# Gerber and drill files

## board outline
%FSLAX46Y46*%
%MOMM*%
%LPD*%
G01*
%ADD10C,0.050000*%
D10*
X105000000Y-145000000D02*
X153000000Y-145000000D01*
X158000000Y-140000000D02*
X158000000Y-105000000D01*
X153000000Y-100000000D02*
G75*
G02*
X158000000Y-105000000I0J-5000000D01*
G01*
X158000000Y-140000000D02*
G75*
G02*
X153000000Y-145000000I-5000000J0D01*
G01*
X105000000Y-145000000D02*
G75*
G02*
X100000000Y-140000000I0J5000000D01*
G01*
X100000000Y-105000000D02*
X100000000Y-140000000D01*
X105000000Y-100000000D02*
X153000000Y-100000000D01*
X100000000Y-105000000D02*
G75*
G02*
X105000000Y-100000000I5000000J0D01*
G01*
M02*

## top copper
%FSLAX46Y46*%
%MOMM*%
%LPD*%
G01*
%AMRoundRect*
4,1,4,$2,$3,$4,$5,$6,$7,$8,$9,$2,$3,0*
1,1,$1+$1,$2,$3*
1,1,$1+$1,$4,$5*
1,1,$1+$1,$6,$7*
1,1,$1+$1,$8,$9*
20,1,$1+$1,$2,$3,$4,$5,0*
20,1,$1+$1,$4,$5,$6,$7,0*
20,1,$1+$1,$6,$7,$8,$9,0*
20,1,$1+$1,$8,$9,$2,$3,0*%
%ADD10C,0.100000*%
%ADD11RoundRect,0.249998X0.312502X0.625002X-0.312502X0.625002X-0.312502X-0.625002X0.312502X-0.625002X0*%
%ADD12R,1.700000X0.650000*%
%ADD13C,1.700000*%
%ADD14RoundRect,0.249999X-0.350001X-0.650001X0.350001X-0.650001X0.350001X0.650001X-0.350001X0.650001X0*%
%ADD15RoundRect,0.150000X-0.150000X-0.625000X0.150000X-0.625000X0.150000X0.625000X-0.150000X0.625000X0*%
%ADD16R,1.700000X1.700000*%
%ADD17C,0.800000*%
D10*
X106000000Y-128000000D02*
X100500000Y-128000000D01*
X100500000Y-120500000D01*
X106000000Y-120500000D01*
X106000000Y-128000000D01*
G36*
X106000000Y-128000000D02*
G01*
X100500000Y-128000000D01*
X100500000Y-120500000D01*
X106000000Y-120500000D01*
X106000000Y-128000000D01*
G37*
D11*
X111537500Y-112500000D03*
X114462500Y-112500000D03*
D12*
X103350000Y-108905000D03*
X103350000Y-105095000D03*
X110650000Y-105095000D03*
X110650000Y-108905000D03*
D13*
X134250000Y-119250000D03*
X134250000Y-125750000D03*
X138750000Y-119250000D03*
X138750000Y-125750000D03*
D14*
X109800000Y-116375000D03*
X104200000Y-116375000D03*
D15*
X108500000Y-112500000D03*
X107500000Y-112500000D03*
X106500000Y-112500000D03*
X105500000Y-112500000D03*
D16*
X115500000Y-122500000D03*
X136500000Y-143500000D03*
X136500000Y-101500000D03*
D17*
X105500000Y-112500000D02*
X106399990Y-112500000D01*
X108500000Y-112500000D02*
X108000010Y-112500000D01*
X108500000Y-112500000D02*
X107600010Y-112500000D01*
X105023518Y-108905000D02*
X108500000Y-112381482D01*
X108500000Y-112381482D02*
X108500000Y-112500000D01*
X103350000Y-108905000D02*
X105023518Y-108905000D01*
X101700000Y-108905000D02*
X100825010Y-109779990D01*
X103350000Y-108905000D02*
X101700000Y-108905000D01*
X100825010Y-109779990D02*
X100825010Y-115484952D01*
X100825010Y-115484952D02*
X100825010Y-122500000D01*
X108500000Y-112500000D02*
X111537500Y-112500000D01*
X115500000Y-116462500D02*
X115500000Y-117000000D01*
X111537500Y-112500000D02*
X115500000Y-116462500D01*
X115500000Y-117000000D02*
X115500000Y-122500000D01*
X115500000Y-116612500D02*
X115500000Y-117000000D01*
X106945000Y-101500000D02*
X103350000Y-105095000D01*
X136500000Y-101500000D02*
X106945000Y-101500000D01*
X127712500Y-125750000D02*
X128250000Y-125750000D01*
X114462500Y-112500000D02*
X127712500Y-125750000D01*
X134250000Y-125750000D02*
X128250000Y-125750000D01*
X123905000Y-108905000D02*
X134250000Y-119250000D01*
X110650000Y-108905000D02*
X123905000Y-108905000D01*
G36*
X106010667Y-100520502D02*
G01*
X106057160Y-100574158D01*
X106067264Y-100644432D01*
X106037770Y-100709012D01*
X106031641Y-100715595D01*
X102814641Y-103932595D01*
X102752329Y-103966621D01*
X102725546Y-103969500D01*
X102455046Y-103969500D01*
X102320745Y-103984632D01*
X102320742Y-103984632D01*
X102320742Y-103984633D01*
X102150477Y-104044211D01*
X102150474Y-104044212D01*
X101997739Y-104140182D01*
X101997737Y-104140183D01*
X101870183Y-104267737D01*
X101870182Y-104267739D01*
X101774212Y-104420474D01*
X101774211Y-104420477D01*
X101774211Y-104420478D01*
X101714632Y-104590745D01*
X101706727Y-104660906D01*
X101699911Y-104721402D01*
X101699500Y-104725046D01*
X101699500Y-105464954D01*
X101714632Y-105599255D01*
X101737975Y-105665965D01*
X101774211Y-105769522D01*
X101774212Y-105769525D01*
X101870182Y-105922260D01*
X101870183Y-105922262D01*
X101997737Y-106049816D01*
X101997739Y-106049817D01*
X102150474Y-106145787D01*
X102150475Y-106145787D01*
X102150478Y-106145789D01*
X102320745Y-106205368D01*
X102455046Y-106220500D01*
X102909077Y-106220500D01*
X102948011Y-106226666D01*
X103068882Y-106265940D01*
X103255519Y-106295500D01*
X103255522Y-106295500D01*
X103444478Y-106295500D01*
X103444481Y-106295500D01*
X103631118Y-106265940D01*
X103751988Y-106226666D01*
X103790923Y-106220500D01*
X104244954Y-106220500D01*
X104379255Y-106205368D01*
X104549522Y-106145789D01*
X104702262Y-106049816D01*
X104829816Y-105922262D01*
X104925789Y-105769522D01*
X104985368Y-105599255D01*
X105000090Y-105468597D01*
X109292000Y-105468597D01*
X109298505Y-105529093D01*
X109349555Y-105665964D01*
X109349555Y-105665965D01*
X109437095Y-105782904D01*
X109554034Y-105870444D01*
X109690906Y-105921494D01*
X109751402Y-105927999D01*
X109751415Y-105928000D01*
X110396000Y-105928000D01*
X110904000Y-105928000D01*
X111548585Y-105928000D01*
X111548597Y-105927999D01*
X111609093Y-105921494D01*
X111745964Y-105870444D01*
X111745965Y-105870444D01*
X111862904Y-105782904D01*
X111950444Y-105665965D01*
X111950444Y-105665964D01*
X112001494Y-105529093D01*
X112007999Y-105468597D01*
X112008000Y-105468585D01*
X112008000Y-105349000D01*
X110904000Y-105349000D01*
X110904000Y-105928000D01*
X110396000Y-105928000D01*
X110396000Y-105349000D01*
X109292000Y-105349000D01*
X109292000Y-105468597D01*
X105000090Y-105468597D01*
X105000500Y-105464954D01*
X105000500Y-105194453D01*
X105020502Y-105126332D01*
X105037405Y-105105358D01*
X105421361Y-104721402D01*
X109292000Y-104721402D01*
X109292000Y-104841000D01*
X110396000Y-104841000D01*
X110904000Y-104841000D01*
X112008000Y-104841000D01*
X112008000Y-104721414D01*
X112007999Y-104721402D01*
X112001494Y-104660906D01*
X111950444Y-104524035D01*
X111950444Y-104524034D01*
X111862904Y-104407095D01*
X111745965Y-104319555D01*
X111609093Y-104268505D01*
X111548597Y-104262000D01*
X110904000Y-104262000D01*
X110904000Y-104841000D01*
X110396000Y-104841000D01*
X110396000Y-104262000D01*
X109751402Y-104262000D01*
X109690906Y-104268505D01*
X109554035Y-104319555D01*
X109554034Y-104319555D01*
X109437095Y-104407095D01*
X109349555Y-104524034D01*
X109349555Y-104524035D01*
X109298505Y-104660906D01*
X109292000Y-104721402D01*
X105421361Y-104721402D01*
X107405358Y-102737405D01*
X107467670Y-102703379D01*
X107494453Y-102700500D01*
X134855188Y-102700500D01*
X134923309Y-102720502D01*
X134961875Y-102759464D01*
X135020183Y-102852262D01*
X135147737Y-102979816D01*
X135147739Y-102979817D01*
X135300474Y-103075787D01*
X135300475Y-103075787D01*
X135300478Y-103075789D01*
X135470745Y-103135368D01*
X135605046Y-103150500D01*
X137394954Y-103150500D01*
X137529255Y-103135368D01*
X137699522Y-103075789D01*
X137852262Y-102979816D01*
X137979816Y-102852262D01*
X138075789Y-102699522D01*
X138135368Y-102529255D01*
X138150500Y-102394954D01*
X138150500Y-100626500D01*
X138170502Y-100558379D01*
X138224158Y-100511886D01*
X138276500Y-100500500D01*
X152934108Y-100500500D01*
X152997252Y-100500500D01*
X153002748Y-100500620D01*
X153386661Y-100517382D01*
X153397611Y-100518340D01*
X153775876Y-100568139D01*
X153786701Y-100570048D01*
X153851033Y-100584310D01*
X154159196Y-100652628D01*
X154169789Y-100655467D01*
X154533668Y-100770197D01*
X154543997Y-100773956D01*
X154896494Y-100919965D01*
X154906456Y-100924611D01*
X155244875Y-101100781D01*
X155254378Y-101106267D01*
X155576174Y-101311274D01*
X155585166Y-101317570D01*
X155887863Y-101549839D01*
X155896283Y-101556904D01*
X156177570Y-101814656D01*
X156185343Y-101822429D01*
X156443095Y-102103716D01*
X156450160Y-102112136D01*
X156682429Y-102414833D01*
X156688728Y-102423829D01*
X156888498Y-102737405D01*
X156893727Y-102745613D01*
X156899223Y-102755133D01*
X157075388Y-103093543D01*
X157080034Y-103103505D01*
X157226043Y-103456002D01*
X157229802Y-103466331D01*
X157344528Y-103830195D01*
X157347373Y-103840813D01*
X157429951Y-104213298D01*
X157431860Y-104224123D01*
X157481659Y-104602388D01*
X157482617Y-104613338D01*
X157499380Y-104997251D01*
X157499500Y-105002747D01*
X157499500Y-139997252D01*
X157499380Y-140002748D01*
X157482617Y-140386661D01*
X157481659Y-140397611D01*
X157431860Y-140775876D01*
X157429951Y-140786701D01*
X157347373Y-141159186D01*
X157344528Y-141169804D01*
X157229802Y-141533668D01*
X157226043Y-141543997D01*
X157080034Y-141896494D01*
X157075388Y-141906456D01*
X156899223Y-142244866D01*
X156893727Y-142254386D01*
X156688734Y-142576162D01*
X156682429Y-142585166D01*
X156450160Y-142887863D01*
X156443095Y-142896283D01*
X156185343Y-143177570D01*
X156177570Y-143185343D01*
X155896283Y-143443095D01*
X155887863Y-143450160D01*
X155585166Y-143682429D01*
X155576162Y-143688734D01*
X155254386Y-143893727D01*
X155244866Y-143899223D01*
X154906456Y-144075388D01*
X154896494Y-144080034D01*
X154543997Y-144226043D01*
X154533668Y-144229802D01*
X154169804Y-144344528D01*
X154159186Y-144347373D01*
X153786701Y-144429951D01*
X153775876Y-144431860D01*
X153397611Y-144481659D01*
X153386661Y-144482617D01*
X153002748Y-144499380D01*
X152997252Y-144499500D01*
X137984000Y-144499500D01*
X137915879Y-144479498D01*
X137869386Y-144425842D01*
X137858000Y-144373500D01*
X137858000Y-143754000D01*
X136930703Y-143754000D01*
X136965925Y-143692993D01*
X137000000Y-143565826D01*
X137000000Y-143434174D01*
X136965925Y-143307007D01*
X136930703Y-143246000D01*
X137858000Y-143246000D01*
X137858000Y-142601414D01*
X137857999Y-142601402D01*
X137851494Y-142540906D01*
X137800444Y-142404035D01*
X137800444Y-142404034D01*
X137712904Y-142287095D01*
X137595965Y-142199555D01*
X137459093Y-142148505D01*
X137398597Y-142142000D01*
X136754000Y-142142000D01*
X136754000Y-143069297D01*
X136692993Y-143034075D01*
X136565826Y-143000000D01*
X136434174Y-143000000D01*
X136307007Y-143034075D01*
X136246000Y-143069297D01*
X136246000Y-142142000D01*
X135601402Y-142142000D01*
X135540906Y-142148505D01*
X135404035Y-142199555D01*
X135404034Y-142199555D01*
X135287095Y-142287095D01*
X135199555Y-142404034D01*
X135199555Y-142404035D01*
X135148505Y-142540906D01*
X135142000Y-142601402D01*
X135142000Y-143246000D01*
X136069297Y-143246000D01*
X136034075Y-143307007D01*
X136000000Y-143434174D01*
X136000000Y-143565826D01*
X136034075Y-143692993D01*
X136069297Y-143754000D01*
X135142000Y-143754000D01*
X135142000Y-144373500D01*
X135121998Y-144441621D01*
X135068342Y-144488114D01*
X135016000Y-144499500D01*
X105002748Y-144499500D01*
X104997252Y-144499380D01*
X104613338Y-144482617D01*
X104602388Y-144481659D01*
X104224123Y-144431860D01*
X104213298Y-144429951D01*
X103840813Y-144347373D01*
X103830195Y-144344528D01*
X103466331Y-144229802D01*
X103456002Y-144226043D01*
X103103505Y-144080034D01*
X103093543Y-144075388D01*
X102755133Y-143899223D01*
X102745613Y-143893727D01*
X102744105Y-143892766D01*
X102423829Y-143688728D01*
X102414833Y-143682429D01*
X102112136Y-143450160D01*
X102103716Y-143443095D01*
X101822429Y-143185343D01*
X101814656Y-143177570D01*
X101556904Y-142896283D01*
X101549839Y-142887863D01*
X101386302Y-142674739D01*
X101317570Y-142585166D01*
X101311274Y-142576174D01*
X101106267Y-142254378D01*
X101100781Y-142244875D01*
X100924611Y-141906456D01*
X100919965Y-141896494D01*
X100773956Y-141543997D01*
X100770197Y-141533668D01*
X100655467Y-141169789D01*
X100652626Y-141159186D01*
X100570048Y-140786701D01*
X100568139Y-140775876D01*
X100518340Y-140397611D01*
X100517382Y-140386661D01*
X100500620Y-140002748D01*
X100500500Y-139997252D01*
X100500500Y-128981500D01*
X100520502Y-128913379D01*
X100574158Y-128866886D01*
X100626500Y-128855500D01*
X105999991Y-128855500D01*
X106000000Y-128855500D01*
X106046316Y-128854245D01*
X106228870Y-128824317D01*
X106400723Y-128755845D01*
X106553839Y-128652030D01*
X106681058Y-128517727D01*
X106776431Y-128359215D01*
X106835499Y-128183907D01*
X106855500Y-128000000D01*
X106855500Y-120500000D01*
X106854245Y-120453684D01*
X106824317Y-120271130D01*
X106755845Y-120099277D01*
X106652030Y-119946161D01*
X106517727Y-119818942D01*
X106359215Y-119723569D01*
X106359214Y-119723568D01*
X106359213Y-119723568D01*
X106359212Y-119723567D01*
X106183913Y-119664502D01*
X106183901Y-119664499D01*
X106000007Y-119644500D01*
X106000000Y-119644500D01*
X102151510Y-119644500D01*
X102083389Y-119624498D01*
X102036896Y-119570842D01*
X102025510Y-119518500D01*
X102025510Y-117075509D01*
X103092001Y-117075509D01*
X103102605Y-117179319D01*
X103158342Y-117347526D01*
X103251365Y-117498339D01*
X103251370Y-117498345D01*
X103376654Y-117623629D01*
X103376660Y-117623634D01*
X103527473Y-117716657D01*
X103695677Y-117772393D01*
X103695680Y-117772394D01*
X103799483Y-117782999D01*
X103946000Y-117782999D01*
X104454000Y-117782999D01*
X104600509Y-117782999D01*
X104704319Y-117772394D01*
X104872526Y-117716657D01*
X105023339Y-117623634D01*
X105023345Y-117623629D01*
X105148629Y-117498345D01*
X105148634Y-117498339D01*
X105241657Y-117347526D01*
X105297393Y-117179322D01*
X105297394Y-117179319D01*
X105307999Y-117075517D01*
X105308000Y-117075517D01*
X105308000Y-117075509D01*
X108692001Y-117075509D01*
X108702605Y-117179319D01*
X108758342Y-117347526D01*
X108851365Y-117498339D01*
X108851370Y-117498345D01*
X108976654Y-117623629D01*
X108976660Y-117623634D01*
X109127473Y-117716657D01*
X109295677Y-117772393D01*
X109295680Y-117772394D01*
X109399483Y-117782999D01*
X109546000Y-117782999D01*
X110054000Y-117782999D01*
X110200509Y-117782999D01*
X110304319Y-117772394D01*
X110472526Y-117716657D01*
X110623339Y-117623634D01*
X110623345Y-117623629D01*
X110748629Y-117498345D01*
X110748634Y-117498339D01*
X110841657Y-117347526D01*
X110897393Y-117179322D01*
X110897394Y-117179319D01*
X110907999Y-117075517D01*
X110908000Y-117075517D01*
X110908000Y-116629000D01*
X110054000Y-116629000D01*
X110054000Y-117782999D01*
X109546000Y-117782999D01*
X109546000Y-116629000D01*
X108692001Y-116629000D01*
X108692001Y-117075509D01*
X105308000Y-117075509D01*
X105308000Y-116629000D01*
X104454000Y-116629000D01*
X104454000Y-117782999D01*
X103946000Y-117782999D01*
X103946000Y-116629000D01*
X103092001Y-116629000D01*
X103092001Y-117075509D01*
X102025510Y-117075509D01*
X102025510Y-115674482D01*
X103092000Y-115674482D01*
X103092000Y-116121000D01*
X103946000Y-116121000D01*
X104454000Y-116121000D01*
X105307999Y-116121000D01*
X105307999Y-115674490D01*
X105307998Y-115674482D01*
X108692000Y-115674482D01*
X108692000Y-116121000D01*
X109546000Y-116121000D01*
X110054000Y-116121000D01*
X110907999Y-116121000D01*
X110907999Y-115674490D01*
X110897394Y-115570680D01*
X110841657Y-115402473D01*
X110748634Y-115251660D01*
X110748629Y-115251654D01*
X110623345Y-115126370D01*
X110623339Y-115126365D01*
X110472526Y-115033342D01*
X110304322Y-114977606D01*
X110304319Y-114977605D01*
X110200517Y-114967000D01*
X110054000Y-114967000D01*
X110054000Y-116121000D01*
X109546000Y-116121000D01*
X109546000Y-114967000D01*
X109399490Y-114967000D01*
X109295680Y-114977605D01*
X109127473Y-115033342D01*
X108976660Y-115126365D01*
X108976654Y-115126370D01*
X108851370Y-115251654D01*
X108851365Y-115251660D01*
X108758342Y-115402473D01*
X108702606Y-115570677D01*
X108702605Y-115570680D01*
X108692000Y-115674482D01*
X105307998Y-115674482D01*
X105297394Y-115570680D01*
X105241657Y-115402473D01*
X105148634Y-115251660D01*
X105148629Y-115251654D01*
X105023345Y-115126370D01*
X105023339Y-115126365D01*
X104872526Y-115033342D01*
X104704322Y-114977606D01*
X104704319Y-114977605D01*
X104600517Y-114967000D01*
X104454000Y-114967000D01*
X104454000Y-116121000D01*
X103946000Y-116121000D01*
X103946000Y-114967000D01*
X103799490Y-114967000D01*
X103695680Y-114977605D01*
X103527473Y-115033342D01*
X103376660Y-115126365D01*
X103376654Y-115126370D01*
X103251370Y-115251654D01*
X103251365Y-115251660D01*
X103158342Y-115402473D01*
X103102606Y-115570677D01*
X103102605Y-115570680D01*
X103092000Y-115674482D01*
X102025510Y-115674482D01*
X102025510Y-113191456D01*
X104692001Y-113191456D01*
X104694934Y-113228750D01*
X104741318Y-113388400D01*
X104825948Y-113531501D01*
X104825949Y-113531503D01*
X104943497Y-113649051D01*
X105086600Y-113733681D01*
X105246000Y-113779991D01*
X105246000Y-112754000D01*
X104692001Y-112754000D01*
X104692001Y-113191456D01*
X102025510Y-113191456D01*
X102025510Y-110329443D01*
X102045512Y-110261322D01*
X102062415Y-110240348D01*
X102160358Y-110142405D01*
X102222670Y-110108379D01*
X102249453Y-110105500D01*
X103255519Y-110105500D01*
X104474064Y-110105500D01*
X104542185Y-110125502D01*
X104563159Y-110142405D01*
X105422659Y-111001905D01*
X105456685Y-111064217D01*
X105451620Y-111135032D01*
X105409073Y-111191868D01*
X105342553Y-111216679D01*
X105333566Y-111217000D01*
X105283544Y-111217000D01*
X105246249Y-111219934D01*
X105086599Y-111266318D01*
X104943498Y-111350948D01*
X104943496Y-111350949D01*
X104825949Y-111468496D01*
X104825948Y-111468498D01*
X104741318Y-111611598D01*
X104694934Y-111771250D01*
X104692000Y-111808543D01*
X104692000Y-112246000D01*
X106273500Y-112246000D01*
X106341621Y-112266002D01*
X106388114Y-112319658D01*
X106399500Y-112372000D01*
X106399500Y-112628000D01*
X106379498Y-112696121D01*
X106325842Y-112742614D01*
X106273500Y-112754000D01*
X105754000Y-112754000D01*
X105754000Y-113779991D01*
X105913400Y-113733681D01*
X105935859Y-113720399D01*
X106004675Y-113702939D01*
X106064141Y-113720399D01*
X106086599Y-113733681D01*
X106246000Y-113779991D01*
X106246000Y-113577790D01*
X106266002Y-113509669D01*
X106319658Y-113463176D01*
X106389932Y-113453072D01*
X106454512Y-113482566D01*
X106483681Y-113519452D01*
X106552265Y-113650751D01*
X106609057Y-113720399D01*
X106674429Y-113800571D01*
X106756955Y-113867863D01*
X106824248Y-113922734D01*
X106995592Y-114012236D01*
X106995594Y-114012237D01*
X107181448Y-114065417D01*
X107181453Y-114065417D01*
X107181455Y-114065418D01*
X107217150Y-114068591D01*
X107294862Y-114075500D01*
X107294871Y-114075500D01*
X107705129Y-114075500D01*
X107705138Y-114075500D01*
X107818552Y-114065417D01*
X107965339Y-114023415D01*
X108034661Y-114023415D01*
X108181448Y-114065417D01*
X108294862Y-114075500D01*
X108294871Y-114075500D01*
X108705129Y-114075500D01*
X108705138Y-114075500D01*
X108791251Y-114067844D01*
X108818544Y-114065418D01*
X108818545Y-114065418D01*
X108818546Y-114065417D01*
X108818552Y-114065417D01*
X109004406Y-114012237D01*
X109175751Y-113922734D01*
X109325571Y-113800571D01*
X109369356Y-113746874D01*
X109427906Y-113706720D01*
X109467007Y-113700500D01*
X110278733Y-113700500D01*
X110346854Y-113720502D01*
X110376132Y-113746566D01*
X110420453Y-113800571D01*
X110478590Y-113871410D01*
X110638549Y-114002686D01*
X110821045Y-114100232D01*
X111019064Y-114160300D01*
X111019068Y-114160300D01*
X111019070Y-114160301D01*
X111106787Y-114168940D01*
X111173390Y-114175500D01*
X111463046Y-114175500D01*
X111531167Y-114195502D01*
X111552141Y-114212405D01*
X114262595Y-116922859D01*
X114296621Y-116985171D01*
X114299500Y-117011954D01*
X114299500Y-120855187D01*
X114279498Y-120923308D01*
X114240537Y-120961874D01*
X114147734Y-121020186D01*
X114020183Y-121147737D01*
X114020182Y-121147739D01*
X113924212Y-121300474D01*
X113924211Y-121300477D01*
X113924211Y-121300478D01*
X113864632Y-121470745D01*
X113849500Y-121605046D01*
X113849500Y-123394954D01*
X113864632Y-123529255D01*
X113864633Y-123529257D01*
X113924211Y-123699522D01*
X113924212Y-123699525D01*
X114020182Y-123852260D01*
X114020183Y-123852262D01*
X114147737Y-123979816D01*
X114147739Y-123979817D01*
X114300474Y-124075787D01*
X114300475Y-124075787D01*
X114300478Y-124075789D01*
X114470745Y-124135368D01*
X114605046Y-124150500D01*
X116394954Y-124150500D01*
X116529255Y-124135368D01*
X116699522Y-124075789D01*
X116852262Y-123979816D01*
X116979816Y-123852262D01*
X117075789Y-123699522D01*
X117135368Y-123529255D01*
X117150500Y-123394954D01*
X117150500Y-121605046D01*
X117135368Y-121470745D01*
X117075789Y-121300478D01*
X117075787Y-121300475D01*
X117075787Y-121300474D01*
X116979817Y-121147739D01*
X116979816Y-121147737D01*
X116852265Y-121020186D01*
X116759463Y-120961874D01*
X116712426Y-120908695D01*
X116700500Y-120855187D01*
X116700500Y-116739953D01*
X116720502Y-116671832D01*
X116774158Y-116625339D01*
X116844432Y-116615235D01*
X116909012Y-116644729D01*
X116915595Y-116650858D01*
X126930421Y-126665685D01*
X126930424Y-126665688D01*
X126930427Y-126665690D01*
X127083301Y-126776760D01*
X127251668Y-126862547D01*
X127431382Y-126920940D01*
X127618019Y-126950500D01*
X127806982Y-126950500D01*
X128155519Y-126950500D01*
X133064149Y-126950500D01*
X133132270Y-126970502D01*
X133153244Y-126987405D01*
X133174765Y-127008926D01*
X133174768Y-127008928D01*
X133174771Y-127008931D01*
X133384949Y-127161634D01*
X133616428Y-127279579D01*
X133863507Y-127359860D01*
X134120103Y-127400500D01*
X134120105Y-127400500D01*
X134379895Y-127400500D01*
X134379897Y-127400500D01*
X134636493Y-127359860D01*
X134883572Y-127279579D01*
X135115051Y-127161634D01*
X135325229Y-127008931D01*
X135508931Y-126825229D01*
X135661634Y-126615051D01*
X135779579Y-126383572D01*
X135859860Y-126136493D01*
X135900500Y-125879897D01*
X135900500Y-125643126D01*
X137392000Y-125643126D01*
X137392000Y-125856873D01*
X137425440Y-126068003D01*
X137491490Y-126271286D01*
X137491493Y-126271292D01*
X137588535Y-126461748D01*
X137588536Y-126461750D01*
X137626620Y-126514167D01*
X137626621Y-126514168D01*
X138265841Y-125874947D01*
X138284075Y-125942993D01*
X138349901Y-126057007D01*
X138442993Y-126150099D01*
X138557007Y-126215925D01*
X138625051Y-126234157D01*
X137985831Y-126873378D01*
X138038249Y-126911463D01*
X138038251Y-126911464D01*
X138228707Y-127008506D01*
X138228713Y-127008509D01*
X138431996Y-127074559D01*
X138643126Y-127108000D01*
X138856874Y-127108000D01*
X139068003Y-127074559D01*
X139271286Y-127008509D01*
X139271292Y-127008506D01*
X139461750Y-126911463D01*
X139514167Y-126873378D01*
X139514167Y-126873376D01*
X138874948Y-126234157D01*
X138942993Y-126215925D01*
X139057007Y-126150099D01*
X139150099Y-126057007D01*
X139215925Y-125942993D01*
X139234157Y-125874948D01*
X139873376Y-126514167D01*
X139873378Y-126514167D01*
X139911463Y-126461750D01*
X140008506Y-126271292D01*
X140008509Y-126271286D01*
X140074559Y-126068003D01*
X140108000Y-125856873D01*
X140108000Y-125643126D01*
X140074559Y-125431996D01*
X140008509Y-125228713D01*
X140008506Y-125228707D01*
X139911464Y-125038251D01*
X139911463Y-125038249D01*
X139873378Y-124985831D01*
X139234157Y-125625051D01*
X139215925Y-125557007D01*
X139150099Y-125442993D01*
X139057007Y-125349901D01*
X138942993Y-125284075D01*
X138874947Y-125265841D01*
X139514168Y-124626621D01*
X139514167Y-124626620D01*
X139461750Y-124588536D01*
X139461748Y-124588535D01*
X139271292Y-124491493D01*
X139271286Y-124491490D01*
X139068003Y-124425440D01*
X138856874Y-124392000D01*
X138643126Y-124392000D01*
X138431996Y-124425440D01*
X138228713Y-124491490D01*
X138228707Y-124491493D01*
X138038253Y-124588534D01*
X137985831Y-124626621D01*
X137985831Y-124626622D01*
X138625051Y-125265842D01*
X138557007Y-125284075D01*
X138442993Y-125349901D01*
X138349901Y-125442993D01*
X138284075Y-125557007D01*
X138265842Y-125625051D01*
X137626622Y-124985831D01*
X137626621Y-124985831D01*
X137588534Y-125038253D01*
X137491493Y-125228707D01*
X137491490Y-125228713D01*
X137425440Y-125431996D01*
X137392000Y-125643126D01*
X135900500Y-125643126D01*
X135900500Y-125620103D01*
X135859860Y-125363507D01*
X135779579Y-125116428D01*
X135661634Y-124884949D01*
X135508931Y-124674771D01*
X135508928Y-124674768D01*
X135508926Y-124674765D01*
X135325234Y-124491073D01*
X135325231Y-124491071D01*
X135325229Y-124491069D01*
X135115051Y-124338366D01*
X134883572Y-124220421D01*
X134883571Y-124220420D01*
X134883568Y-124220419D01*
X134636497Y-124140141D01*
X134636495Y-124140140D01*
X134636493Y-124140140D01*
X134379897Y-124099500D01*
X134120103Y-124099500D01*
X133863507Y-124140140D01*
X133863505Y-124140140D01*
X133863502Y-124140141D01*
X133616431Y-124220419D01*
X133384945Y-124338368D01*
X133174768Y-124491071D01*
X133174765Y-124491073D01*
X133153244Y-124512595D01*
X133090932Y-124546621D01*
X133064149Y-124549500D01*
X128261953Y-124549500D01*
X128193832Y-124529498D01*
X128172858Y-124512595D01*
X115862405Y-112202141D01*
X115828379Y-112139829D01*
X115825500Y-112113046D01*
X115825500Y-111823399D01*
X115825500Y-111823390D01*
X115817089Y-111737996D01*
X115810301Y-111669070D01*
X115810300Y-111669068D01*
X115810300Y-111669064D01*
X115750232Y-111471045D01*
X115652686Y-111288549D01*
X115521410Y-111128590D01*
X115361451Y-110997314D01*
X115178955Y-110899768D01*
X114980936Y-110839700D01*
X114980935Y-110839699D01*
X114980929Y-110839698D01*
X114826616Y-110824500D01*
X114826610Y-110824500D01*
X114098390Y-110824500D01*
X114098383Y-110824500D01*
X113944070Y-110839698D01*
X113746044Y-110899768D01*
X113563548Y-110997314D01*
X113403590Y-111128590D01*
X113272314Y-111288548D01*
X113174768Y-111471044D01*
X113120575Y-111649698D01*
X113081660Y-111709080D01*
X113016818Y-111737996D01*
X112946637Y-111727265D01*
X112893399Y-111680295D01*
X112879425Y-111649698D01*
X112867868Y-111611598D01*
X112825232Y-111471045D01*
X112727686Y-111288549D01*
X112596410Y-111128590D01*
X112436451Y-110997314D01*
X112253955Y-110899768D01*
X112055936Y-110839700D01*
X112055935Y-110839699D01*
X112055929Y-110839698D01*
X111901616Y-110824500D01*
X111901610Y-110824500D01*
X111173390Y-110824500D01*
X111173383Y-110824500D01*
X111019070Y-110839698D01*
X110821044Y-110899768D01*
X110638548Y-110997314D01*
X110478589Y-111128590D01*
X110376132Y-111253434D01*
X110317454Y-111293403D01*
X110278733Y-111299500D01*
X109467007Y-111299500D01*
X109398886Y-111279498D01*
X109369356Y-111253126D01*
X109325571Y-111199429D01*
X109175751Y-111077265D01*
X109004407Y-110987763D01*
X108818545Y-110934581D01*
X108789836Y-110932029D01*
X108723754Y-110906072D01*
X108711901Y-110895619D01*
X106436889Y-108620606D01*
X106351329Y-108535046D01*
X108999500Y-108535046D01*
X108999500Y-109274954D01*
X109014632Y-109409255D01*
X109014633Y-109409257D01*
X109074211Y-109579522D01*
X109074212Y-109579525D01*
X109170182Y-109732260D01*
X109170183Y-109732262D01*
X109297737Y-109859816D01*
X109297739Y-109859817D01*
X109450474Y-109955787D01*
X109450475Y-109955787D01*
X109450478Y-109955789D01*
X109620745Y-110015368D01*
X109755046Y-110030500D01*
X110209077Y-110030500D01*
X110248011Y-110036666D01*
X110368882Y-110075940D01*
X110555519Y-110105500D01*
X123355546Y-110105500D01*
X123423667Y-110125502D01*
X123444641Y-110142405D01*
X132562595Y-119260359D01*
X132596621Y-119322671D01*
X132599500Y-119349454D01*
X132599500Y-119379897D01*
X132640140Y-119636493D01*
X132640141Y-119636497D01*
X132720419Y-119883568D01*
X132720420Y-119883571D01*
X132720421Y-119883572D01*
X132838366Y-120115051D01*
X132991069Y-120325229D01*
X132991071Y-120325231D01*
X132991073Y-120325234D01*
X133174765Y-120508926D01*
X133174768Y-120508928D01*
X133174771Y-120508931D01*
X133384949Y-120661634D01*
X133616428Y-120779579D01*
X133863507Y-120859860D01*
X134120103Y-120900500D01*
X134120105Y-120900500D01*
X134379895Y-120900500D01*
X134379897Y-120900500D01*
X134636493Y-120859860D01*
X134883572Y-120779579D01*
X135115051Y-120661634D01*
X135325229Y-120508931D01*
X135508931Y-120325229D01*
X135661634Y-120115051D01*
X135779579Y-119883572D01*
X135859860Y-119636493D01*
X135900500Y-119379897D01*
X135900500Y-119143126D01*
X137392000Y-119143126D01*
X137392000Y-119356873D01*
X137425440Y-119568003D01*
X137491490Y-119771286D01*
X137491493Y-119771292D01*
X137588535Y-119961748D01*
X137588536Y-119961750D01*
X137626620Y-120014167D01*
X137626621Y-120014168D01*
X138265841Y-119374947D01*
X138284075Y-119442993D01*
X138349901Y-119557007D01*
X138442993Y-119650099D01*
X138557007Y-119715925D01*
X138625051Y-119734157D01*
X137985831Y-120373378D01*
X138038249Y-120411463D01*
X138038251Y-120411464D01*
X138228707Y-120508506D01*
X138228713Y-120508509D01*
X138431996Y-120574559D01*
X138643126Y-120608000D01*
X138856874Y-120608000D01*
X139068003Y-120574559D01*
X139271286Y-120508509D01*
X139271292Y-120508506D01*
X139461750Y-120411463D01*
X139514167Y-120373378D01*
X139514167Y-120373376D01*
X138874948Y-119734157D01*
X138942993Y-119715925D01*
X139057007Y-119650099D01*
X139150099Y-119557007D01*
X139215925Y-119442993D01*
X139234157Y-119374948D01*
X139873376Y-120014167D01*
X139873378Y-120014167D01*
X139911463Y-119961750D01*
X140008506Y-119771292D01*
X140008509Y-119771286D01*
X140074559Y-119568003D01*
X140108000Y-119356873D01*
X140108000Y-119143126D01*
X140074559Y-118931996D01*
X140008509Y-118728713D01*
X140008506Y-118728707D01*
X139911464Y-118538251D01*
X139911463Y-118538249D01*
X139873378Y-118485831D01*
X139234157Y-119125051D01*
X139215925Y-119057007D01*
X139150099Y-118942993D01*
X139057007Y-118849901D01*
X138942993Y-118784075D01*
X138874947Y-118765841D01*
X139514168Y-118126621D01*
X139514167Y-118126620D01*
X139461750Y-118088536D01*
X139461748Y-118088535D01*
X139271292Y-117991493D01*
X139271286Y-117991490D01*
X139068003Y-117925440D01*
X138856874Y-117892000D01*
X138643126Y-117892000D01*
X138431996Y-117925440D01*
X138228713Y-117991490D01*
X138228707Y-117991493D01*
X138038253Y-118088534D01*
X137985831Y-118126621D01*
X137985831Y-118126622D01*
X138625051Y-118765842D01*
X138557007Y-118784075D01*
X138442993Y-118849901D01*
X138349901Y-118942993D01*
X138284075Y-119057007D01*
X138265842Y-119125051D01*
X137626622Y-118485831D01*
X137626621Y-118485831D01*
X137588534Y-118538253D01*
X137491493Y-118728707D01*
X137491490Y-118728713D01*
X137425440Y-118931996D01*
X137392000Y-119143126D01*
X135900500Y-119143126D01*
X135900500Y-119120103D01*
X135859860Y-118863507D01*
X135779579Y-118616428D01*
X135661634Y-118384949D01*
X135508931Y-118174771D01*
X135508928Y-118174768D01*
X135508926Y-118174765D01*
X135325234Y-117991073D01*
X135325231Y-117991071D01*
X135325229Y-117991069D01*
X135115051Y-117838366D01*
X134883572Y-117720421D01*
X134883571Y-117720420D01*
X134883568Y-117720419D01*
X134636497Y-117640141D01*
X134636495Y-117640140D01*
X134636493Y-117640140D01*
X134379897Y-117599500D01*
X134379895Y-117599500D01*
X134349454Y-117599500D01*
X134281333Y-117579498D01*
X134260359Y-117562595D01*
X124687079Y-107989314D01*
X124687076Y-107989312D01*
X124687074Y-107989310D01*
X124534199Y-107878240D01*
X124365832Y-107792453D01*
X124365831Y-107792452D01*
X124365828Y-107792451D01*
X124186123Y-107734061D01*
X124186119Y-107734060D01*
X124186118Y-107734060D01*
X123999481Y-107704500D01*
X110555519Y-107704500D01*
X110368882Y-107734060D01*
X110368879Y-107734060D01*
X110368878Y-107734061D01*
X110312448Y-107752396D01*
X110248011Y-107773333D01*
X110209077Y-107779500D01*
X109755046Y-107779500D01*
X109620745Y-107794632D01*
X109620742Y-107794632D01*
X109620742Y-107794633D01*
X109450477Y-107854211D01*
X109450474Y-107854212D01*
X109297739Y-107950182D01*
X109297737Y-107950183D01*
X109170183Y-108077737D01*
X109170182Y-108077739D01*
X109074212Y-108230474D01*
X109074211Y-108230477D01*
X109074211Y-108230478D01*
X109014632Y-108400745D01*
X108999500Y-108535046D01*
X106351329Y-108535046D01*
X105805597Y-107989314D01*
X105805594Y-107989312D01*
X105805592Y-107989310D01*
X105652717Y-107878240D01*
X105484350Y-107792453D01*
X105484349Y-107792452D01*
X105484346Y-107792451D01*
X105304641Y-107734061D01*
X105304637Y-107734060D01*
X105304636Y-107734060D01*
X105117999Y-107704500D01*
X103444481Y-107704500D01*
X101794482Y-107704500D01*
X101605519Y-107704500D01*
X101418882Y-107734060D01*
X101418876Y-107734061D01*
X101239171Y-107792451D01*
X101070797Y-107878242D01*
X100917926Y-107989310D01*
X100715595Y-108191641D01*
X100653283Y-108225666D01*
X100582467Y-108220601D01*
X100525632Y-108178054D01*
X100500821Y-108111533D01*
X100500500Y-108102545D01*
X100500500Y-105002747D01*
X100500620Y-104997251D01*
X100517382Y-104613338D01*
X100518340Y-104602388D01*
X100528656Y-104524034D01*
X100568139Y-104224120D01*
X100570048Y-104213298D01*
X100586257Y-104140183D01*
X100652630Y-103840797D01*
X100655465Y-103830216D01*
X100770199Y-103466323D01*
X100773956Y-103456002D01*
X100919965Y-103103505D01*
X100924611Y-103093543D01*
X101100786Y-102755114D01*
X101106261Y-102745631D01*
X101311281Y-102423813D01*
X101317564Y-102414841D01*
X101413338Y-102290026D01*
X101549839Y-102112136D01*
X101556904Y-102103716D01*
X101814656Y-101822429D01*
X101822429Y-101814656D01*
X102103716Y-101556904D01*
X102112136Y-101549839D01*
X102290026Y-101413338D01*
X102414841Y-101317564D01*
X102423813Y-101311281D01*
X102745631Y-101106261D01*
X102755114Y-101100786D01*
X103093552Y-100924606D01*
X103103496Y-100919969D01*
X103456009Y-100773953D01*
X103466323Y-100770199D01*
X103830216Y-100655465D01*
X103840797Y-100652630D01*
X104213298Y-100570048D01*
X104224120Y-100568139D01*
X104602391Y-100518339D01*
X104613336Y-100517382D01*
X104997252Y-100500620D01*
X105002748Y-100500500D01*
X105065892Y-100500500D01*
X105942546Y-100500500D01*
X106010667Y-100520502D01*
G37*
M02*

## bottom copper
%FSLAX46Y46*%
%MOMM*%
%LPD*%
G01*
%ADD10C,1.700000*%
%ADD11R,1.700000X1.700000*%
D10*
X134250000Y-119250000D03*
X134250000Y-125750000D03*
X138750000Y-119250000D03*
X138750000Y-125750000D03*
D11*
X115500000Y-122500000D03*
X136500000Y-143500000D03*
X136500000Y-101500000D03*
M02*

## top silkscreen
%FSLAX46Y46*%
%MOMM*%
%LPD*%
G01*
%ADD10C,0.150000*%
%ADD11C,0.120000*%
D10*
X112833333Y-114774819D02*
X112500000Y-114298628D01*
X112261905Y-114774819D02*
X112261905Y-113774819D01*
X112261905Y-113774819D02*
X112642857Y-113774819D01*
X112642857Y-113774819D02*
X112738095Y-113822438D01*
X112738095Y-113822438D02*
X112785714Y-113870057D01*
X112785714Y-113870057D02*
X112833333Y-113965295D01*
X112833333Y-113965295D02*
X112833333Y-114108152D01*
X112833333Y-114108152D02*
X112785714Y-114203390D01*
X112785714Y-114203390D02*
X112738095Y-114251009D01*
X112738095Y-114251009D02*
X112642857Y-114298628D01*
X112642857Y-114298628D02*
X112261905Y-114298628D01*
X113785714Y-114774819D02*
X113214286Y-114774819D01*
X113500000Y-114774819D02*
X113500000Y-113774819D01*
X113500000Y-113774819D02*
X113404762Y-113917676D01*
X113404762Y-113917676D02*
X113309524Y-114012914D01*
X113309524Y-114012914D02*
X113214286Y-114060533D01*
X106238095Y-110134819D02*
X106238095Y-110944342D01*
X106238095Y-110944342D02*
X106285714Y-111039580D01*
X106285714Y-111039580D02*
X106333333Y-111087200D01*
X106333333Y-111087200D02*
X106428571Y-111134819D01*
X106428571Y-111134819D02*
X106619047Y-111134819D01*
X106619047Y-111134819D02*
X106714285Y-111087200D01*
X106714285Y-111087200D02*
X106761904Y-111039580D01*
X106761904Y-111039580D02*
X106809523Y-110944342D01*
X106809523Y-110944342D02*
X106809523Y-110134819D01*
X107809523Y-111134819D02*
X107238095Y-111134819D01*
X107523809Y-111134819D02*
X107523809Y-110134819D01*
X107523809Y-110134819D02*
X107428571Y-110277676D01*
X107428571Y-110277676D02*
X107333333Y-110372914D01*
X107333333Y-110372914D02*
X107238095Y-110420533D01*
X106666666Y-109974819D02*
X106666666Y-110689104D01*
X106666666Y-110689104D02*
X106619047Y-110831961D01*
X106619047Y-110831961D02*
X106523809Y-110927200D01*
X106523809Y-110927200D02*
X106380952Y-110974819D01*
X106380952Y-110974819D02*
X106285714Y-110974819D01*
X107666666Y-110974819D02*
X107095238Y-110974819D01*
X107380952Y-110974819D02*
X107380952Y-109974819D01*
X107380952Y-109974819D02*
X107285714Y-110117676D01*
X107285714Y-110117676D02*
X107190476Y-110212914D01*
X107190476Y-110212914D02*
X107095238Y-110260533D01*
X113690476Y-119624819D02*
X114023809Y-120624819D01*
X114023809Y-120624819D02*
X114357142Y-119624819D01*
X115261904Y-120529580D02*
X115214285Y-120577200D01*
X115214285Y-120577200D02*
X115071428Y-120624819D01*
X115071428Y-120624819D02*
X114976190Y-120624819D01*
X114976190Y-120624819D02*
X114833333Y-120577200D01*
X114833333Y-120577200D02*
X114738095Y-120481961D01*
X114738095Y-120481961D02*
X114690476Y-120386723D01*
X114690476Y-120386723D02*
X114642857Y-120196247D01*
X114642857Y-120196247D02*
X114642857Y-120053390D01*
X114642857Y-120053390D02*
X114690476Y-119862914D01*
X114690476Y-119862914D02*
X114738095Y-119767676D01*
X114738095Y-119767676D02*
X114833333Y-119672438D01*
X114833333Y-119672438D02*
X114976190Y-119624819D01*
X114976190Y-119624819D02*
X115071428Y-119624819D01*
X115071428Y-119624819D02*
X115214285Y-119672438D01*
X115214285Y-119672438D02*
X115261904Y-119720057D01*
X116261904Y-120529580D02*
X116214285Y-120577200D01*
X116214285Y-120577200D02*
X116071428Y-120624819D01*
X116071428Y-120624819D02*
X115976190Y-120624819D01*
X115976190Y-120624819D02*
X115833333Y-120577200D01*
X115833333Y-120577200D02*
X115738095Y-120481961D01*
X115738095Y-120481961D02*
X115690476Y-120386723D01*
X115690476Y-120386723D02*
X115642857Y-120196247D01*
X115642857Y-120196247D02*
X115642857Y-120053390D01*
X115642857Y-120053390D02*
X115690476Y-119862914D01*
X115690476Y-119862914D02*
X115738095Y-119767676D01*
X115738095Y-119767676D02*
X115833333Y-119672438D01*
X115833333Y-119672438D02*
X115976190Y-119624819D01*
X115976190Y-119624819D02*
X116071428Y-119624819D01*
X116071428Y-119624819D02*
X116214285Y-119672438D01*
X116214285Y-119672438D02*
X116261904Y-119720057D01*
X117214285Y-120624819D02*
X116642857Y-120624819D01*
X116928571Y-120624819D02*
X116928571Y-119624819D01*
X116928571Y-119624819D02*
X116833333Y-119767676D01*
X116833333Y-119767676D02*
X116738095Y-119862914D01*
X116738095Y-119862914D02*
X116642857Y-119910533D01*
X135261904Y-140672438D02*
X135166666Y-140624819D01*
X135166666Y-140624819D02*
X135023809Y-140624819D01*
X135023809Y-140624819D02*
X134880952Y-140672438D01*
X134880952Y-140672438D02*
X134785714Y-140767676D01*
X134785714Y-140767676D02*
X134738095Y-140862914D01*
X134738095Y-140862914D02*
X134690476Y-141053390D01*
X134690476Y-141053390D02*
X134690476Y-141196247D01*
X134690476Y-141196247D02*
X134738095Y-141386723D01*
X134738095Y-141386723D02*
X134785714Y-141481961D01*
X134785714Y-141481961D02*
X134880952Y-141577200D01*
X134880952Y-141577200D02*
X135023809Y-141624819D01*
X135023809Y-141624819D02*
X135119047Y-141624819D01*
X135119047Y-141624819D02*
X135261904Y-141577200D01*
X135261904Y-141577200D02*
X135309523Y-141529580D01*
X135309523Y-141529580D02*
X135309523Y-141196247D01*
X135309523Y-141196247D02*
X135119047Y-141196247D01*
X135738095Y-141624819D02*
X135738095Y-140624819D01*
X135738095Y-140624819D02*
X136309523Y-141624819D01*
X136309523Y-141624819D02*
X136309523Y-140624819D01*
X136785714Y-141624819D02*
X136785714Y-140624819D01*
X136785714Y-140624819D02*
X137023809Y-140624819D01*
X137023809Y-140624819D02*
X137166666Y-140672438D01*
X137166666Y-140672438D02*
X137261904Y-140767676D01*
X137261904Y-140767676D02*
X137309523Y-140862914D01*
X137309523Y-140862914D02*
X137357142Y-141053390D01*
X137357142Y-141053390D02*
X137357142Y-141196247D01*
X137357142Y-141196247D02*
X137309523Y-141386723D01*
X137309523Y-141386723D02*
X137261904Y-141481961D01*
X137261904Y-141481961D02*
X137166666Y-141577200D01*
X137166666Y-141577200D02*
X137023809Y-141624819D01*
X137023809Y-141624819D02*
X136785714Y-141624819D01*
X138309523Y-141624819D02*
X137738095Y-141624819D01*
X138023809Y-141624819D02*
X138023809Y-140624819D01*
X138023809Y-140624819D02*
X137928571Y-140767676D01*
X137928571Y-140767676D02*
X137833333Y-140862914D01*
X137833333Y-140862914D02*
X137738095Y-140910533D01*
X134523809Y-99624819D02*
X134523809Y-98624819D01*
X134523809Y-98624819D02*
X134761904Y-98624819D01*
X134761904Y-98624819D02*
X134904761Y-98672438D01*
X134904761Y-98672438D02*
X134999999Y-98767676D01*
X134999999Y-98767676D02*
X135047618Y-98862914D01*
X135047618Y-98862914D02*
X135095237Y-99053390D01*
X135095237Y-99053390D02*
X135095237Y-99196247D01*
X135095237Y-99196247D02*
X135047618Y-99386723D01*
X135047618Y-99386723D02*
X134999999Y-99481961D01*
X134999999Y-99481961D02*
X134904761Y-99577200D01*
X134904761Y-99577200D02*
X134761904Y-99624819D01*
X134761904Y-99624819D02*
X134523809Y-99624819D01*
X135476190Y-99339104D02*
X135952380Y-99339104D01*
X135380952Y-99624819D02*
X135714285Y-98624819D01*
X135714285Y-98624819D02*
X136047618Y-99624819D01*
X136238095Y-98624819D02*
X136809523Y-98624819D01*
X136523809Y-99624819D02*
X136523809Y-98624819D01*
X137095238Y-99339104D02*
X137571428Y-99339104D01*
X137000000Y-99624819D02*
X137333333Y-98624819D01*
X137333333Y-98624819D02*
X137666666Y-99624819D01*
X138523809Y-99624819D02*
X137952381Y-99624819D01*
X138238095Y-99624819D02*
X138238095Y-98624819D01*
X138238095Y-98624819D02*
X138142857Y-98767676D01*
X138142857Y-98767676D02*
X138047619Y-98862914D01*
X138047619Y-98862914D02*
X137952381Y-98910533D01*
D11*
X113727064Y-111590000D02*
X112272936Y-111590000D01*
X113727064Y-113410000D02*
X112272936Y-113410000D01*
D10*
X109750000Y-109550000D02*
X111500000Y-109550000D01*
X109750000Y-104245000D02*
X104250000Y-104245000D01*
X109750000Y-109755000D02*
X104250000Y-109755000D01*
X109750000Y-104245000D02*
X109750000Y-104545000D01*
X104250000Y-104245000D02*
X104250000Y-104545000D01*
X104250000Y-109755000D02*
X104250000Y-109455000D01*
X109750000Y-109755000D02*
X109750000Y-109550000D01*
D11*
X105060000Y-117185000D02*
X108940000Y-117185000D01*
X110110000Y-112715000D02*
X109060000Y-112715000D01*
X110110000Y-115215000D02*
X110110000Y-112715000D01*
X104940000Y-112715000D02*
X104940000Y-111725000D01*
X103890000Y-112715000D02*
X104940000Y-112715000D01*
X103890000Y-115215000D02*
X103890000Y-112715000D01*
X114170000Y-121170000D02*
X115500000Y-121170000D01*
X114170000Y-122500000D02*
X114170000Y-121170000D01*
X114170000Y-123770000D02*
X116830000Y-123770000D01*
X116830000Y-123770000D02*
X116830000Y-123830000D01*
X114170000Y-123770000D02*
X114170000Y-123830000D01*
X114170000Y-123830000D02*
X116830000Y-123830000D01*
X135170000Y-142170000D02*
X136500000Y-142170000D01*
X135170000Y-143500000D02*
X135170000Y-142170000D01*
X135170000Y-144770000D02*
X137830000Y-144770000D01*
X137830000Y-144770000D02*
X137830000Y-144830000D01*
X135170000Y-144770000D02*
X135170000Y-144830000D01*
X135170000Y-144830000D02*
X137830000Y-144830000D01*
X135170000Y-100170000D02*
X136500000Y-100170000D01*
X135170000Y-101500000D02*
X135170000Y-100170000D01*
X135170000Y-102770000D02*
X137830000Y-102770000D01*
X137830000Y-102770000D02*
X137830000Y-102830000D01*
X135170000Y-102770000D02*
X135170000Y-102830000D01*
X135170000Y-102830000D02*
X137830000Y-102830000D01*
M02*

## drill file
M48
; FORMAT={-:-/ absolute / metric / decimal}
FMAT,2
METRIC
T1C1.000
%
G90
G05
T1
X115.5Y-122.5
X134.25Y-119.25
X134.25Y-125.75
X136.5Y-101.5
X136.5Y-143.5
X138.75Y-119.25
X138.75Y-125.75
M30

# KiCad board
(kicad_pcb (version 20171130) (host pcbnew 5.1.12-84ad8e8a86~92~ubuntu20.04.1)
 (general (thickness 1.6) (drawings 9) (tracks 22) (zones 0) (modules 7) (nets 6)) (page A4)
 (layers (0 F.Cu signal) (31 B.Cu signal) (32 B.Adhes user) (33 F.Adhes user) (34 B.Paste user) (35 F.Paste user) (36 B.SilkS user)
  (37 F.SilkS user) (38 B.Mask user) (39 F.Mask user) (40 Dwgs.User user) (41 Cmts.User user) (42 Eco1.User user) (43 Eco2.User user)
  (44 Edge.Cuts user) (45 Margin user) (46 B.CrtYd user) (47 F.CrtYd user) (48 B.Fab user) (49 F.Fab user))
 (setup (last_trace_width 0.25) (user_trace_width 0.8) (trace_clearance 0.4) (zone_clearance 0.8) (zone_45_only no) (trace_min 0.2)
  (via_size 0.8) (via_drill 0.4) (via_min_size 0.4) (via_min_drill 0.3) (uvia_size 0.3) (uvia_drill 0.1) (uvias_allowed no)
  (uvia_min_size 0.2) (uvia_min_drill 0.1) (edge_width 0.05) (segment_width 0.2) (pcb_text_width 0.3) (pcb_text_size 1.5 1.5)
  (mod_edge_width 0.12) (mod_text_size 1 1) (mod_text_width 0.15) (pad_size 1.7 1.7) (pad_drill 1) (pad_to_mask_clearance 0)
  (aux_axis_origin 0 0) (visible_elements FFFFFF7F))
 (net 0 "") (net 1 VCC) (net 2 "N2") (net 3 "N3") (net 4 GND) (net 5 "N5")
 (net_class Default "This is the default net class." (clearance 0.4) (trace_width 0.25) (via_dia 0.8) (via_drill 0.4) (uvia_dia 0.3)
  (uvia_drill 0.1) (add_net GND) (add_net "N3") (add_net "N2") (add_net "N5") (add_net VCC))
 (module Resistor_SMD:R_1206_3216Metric (layer F.Cu) (at 113 112.5 180)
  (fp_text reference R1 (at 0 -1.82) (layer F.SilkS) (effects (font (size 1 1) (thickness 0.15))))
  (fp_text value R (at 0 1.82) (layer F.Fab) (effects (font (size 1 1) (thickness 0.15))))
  (fp_line (start -0.727064 0.91) (end 0.727064 0.91) (layer F.SilkS) (width 0.12))
  (fp_line (start -0.727064 -0.91) (end 0.727064 -0.91) (layer F.SilkS) (width 0.12))
  (pad 2 smd roundrect (at 1.4625 0 180) (size 1.125 1.75) (layers F.Cu F.Paste F.Mask) (roundrect_rratio 0.2222204444444444) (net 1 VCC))
  (pad 1 smd roundrect (at -1.4625 0 180) (size 1.125 1.75) (layers F.Cu F.Paste F.Mask) (roundrect_rratio 0.2222204444444444) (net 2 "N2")))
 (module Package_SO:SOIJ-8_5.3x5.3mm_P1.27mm (layer F.Cu) (at 107 107 180)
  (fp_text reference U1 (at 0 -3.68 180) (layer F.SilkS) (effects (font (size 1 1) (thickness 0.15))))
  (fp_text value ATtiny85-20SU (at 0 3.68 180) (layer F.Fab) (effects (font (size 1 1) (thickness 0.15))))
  (fp_line (start -2.75 -2.55) (end -4.5 -2.55) (layer F.SilkS) (width 0.15))
  (fp_line (start -2.75 2.755) (end 2.75 2.755) (layer F.SilkS) (width 0.15))
  (fp_line (start -2.75 -2.755) (end 2.75 -2.755) (layer F.SilkS) (width 0.15))
  (fp_line (start -2.75 2.755) (end -2.75 2.455) (layer F.SilkS) (width 0.15))
  (fp_line (start 2.75 2.755) (end 2.75 2.455) (layer F.SilkS) (width 0.15))
  (fp_line (start 2.75 -2.755) (end 2.75 -2.455) (layer F.SilkS) (width 0.15))
  (fp_line (start -2.75 -2.755) (end -2.75 -2.55) (layer F.SilkS) (width 0.15))
  (pad 8 smd rect (at 3.65 -1.905 180) (size 1.7 0.65) (layers F.Cu F.Paste F.Mask) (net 1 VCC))
  (pad 5 smd rect (at 3.65 1.905 180) (size 1.7 0.65) (layers F.Cu F.Paste F.Mask) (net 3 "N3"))
  (pad 4 smd rect (at -3.65 1.905 180) (size 1.7 0.65) (layers F.Cu F.Paste F.Mask) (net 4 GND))
  (pad 1 smd rect (at -3.65 -1.905 180) (size 1.7 0.65) (layers F.Cu F.Paste F.Mask) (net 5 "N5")))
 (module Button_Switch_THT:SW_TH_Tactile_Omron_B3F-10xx (layer B.Cu) (at 136.5 122.5 270)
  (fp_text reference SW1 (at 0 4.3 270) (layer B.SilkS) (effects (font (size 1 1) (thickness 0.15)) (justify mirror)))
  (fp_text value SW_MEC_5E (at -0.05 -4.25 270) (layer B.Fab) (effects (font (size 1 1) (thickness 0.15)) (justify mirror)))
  (pad 1 thru_hole circle (at -3.25 2.25 270) (size 1.7 1.7) (drill 1) (layers *.Cu *.Mask) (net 5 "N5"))
  (pad 2 thru_hole circle (at 3.25 2.25 270) (size 1.7 1.7) (drill 1) (layers *.Cu *.Mask) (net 2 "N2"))
  (pad 3 thru_hole circle (at -3.25 -2.25 270) (size 1.7 1.7) (drill 1) (layers *.Cu *.Mask) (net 4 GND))
  (pad 4 thru_hole circle (at 3.25 -2.25 270) (size 1.7 1.7) (drill 1) (layers *.Cu *.Mask) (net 4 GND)))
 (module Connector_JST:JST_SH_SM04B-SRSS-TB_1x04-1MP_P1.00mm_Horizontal (layer F.Cu) (at 107 114.5)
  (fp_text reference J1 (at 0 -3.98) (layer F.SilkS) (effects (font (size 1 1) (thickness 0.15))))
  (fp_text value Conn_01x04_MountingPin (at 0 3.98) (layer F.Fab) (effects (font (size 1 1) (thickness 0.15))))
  (fp_line (start -1.94 2.685) (end 1.94 2.685) (layer F.SilkS) (width 0.12))
  (fp_line (start 3.11 -1.785) (end 2.06 -1.785) (layer F.SilkS) (width 0.12))
  (fp_line (start 3.11 0.715) (end 3.11 -1.785) (layer F.SilkS) (width 0.12))
  (fp_line (start -2.06 -1.785) (end -2.06 -2.775) (layer F.SilkS) (width 0.12))
  (fp_line (start -3.11 -1.785) (end -2.06 -1.785) (layer F.SilkS) (width 0.12))
  (fp_line (start -3.11 0.715) (end -3.11 -1.785) (layer F.SilkS) (width 0.12))
  (pad MP smd roundrect (at 2.8 1.875) (size 1.2 1.8) (layers F.Cu F.Paste F.Mask) (roundrect_rratio 0.2083325) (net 4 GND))
  (pad MP smd roundrect (at -2.8 1.875) (size 1.2 1.8) (layers F.Cu F.Paste F.Mask) (roundrect_rratio 0.2083325) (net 4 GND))
  (pad 4 smd roundrect (at 1.5 -2) (size 0.6 1.55) (layers F.Cu F.Paste F.Mask) (roundrect_rratio 0.25) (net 1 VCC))
  (pad 3 smd roundrect (at 0.5 -2) (size 0.6 1.55) (layers F.Cu F.Paste F.Mask) (roundrect_rratio 0.25) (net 1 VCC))
  (pad 2 smd roundrect (at -0.5 -2) (size 0.6 1.55) (layers F.Cu F.Paste F.Mask) (roundrect_rratio 0.25) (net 4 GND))
  (pad 1 smd roundrect (at -1.5 -2) (size 0.6 1.55) (layers F.Cu F.Paste F.Mask) (roundrect_rratio 0.25) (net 4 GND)))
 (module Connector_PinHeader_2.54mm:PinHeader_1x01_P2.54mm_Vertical (layer F.Cu) (at 115.5 122.5)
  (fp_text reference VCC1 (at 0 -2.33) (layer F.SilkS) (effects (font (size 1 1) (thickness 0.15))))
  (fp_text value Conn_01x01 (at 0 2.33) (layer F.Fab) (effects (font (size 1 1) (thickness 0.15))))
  (fp_line (start -1.33 -1.33) (end 0 -1.33) (layer F.SilkS) (width 0.12))
  (fp_line (start -1.33 0) (end -1.33 -1.33) (layer F.SilkS) (width 0.12))
  (fp_line (start -1.33 1.27) (end 1.33 1.27) (layer F.SilkS) (width 0.12))
  (fp_line (start 1.33 1.27) (end 1.33 1.33) (layer F.SilkS) (width 0.12))
  (fp_line (start -1.33 1.27) (end -1.33 1.33) (layer F.SilkS) (width 0.12))
  (fp_line (start -1.33 1.33) (end 1.33 1.33) (layer F.SilkS) (width 0.12))
  (pad 1 thru_hole rect (at 0 0) (size 1.7 1.7) (drill 1) (layers *.Cu *.Mask) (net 1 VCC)))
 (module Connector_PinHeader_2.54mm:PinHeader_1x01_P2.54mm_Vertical (layer F.Cu) (at 136.5 143.5)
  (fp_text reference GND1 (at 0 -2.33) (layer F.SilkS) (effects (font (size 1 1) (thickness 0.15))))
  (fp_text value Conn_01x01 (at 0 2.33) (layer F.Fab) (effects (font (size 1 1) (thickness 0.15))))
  (fp_line (start -1.33 -1.33) (end 0 -1.33) (layer F.SilkS) (width 0.12))
  (fp_line (start -1.33 0) (end -1.33 -1.33) (layer F.SilkS) (width 0.12))
  (fp_line (start -1.33 1.27) (end 1.33 1.27) (layer F.SilkS) (width 0.12))
  (fp_line (start 1.33 1.27) (end 1.33 1.33) (layer F.SilkS) (width 0.12))
  (fp_line (start -1.33 1.27) (end -1.33 1.33) (layer F.SilkS) (width 0.12))
  (fp_line (start -1.33 1.33) (end 1.33 1.33) (layer F.SilkS) (width 0.12))
  (pad 1 thru_hole rect (at 0 0) (size 1.7 1.7) (drill 1) (layers *.Cu *.Mask) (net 4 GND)))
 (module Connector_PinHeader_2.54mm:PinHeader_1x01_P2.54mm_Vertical (layer F.Cu) (at 136.5 101.5)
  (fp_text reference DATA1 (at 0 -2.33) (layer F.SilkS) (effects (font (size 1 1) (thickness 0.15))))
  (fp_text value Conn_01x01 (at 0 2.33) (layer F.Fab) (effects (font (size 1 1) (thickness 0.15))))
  (fp_line (start -1.33 -1.33) (end 0 -1.33) (layer F.SilkS) (width 0.12))
  (fp_line (start -1.33 0) (end -1.33 -1.33) (layer F.SilkS) (width 0.12))
  (fp_line (start -1.33 1.27) (end 1.33 1.27) (layer F.SilkS) (width 0.12))
  (fp_line (start 1.33 1.27) (end 1.33 1.33) (layer F.SilkS) (width 0.12))
  (fp_line (start -1.33 1.27) (end -1.33 1.33) (layer F.SilkS) (width 0.12))
  (fp_line (start -1.33 1.33) (end 1.33 1.33) (layer F.SilkS) (width 0.12))
  (pad 1 thru_hole rect (at 0 0) (size 1.7 1.7) (drill 1) (layers *.Cu *.Mask) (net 3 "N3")))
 (gr_poly (pts (xy 106 128) (xy 100.5 128) (xy 100.5 120.5) (xy 106 120.5)) (layer F.Cu) (width 0.1))
 (gr_line (start 105 145) (end 153 145) (layer Edge.Cuts) (width 0.05))
 (gr_line (start 158 140) (end 158 105) (layer Edge.Cuts) (width 0.05))
 (gr_arc (start 153 105) (end 158 105) (angle -90) (layer Edge.Cuts) (width 0.05))
 (gr_arc (start 153 140) (end 153 145) (angle -90) (layer Edge.Cuts) (width 0.05))
 (gr_arc (start 105 140) (end 100 140) (angle -90) (layer Edge.Cuts) (width 0.05))
 (gr_line (start 100 105) (end 100 140) (layer Edge.Cuts) (width 0.05))
 (gr_line (start 105 100) (end 153 100) (layer Edge.Cuts) (width 0.05))
 (gr_arc (start 105 105) (end 105 100) (angle -90) (layer Edge.Cuts) (width 0.05))
 (segment (start 105.5 112.5) (end 106.39999 112.5) (width 0.8) (layer F.Cu) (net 4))
 (segment (start 108.5 112.5) (end 108.00001 112.5) (width 0.8) (layer F.Cu) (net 1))
 (segment (start 108.5 112.5) (end 107.60001 112.5) (width 0.8) (layer F.Cu) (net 1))
 (segment (start 105.023518 108.905) (end 108.5 112.381482) (width 0.8) (layer F.Cu) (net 1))
 (segment (start 108.5 112.381482) (end 108.5 112.5) (width 0.8) (layer F.Cu) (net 1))
 (segment (start 103.35 108.905) (end 105.023518 108.905) (width 0.8) (layer F.Cu) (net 1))
 (segment (start 101.7 108.905) (end 100.82501 109.77999) (width 0.8) (layer F.Cu) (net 1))
 (segment (start 103.35 108.905) (end 101.7 108.905) (width 0.8) (layer F.Cu) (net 1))
 (segment (start 100.82501 109.77999) (end 100.82501 115.484952) (width 0.8) (layer F.Cu) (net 1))
 (segment (start 100.82501 115.484952) (end 100.82501 122.5) (width 0.8) (layer F.Cu) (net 1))
 (segment (start 108.5 112.5) (end 111.5375 112.5) (width 0.8) (layer F.Cu) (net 1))
 (segment (start 115.5 116.4625) (end 115.5 117) (width 0.8) (layer F.Cu) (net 1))
 (segment (start 111.5375 112.5) (end 115.5 116.4625) (width 0.8) (layer F.Cu) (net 1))
 (segment (start 115.5 117) (end 115.5 122.5) (width 0.8) (layer F.Cu) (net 1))
 (segment (start 115.5 116.6125) (end 115.5 117) (width 0.8) (layer F.Cu) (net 1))
 (segment (start 106.945 101.5) (end 103.35 105.095) (width 0.8) (layer F.Cu) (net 3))
 (segment (start 136.5 101.5) (end 106.945 101.5) (width 0.8) (layer F.Cu) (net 3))
 (segment (start 127.7125 125.75) (end 128.25 125.75) (width 0.8) (layer F.Cu) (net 2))
 (segment (start 114.4625 112.5) (end 127.7125 125.75) (width 0.8) (layer F.Cu) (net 2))
 (segment (start 134.25 125.75) (end 128.25 125.75) (width 0.8) (layer F.Cu) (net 2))
 (segment (start 123.905 108.905) (end 134.25 119.25) (width 0.8) (layer F.Cu) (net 5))
 (segment (start 110.65 108.905) (end 123.905 108.905) (width 0.8) (layer F.Cu) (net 5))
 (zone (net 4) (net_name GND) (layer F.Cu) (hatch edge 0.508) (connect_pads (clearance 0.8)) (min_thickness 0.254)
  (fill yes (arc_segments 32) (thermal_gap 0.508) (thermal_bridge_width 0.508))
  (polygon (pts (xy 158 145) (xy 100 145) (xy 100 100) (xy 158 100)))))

